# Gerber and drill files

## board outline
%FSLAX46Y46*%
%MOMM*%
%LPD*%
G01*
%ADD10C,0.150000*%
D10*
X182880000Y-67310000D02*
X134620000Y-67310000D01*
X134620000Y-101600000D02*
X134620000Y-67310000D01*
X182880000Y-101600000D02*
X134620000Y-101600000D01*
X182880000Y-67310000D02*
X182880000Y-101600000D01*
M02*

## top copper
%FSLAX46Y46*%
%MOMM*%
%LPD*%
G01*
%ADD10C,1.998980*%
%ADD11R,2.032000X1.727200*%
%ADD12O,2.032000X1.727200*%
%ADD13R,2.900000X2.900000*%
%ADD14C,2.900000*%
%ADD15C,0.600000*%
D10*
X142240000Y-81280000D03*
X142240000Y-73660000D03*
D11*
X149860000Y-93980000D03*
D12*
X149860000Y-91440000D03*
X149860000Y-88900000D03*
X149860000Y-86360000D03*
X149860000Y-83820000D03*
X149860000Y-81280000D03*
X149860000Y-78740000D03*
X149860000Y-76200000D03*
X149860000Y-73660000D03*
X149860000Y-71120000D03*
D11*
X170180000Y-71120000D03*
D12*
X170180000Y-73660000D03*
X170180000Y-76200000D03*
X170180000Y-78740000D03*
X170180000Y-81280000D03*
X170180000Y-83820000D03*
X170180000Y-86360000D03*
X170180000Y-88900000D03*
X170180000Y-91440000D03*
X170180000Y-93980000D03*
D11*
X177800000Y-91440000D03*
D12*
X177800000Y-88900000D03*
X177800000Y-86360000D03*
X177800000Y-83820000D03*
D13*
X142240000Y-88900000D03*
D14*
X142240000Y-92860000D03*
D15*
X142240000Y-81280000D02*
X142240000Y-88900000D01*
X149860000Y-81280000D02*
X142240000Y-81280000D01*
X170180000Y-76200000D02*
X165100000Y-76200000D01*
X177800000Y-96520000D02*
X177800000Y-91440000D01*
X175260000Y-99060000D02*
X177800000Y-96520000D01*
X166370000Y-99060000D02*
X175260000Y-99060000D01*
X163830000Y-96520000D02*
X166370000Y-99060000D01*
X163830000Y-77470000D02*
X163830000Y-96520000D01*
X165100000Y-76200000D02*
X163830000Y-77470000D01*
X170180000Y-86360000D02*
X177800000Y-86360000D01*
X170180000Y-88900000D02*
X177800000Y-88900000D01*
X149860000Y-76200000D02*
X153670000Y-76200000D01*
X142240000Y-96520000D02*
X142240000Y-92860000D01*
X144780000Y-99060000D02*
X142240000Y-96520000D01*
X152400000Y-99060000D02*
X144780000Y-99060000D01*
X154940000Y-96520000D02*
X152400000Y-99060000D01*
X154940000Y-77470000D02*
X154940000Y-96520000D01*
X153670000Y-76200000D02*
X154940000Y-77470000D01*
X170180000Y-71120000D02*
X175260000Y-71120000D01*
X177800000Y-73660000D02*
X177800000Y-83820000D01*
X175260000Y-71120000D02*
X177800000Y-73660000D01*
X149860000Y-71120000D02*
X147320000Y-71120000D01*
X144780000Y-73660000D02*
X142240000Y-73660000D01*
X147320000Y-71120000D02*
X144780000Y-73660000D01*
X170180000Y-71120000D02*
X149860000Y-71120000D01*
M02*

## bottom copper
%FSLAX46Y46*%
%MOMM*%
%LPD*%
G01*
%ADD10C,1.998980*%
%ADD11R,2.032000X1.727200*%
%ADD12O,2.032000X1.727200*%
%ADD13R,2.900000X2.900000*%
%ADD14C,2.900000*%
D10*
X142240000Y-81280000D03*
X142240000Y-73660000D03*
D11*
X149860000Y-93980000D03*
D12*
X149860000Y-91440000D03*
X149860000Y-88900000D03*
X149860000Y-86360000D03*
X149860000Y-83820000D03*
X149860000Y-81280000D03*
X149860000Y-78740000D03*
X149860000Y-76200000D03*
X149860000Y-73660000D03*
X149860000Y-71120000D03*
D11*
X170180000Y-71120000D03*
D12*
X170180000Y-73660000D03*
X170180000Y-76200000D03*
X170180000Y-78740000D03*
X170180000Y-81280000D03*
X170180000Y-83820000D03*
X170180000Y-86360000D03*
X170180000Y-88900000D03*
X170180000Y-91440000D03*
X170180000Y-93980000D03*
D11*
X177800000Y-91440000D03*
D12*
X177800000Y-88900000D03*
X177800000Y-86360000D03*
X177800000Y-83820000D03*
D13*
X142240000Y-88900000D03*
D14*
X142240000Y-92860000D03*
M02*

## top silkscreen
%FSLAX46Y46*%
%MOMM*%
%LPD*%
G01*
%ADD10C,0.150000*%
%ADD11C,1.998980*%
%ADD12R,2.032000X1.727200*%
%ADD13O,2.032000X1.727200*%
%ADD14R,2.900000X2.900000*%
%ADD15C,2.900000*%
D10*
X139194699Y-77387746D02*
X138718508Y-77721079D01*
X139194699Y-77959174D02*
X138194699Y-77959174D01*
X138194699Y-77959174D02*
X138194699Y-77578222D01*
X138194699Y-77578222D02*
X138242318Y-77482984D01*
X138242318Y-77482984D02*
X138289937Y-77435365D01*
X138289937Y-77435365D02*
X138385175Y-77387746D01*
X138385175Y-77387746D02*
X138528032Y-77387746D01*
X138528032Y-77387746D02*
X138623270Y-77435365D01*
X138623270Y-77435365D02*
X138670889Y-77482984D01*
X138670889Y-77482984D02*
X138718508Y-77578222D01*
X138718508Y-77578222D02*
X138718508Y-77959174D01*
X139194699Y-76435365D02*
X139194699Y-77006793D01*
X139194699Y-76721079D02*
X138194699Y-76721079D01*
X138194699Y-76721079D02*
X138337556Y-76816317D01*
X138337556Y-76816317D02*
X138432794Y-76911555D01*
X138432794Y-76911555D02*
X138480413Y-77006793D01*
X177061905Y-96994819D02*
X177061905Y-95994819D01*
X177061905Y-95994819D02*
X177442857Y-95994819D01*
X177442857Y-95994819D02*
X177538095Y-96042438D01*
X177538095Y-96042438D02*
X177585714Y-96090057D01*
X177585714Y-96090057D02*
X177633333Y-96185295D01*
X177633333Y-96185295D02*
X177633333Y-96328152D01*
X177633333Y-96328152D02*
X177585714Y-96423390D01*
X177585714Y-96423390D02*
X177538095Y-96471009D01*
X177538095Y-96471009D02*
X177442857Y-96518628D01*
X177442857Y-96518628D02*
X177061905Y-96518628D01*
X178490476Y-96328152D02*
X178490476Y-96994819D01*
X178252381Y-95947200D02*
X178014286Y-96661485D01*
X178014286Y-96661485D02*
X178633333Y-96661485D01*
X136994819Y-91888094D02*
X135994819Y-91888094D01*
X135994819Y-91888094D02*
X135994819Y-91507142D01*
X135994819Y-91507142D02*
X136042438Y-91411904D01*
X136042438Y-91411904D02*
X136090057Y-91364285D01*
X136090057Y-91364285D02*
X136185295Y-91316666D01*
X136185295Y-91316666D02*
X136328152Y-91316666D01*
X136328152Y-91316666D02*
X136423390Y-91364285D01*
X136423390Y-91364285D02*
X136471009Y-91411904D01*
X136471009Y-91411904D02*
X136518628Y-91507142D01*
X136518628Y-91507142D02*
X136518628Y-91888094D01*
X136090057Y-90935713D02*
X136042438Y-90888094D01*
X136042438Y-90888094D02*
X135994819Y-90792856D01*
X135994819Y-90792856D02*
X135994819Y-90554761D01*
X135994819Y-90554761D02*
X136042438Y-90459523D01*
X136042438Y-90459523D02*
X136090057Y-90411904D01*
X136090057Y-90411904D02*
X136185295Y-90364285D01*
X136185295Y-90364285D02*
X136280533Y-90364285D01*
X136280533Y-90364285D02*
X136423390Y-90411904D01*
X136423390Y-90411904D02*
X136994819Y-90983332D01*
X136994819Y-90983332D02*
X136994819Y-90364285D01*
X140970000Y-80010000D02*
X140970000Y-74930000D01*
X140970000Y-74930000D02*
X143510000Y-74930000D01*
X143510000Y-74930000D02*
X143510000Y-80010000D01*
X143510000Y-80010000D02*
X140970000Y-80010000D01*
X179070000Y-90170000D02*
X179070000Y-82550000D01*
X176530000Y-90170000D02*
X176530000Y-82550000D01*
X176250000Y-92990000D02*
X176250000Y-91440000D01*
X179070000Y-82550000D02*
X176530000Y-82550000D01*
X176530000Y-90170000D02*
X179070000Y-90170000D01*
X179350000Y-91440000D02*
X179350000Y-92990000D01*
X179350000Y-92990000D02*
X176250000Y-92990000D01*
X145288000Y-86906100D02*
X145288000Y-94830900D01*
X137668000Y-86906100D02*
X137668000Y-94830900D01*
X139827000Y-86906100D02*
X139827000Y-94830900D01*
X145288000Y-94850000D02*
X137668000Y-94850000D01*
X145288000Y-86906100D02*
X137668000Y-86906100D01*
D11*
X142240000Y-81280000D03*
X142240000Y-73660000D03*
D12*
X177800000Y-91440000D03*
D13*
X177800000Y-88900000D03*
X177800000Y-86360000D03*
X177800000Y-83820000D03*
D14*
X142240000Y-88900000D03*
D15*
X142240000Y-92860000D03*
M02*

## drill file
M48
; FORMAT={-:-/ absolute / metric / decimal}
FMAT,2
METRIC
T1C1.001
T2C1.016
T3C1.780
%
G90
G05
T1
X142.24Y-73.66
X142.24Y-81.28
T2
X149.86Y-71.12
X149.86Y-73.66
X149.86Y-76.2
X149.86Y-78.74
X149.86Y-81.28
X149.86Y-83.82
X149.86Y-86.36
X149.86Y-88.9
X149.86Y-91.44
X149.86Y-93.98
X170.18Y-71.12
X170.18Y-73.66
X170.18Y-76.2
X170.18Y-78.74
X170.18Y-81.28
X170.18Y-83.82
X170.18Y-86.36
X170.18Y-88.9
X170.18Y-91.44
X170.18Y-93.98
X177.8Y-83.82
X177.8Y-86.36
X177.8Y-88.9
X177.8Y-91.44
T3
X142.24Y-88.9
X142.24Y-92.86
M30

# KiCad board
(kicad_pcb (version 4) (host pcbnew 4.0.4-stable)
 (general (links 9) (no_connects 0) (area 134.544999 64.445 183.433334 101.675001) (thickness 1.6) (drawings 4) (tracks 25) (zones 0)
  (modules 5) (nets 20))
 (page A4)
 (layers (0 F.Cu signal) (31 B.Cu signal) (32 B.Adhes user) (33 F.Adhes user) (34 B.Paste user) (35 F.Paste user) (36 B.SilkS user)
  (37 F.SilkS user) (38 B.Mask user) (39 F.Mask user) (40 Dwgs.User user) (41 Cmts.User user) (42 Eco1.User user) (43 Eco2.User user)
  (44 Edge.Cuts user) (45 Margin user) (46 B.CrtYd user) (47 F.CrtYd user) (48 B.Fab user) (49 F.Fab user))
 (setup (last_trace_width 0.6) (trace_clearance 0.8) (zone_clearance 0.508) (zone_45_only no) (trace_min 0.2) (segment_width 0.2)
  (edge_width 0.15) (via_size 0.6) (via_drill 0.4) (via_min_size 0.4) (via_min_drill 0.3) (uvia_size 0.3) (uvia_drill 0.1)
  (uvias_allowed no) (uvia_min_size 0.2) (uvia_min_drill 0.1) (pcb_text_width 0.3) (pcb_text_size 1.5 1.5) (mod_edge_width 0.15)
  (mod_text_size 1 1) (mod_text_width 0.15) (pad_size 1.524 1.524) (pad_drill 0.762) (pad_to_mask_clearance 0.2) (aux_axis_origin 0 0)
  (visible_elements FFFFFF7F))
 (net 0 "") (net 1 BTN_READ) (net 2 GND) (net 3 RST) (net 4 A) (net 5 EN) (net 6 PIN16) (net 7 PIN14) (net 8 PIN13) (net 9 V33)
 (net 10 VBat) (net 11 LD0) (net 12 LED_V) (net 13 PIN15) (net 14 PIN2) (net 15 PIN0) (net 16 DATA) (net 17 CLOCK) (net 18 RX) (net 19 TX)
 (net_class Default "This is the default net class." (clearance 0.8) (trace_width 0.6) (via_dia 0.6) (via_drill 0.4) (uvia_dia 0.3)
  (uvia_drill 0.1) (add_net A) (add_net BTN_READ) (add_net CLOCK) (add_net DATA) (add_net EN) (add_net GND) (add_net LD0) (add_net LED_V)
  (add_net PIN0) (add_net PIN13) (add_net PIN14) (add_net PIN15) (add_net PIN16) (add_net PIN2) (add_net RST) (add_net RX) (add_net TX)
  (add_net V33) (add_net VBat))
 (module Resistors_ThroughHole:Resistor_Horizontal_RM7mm (layer F.Cu) (at 142.24 81.28 90)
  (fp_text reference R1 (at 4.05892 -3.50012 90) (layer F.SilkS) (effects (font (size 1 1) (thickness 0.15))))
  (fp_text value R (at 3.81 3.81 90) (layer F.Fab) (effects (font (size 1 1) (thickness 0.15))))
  (fp_line (start 1.27 -1.27) (end 6.35 -1.27) (layer F.SilkS) (width 0.15))
  (fp_line (start 6.35 -1.27) (end 6.35 1.27) (layer F.SilkS) (width 0.15))
  (fp_line (start 6.35 1.27) (end 1.27 1.27) (layer F.SilkS) (width 0.15))
  (fp_line (start 1.27 1.27) (end 1.27 -1.27) (layer F.SilkS) (width 0.15))
  (pad 1 thru_hole circle (at 0 0 90) (size 1.99898 1.99898) (drill 1.00076) (layers *.Cu *.SilkS *.Mask) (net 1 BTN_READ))
  (pad 2 thru_hole circle (at 7.62 0 90) (size 1.99898 1.99898) (drill 1.00076) (layers *.Cu *.SilkS *.Mask) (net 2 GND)))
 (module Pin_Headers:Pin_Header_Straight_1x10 (layer B.Cu) (at 149.86 93.98)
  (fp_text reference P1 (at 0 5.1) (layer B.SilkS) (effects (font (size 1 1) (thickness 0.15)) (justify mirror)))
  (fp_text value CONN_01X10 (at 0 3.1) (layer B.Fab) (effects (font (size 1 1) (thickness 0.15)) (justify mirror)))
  (pad 1 thru_hole rect (at 0 0) (size 2.032 1.7272) (drill 1.016) (layers *.Cu *.Mask B.SilkS) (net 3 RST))
  (pad 2 thru_hole oval (at 0 -2.54) (size 2.032 1.7272) (drill 1.016) (layers *.Cu *.Mask B.SilkS) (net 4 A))
  (pad 3 thru_hole oval (at 0 -5.08) (size 2.032 1.7272) (drill 1.016) (layers *.Cu *.Mask B.SilkS) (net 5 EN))
  (pad 4 thru_hole oval (at 0 -7.62) (size 2.032 1.7272) (drill 1.016) (layers *.Cu *.Mask B.SilkS) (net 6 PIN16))
  (pad 5 thru_hole oval (at 0 -10.16) (size 2.032 1.7272) (drill 1.016) (layers *.Cu *.Mask B.SilkS) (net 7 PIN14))
  (pad 6 thru_hole oval (at 0 -12.7) (size 2.032 1.7272) (drill 1.016) (layers *.Cu *.Mask B.SilkS) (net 1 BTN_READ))
  (pad 7 thru_hole oval (at 0 -15.24) (size 2.032 1.7272) (drill 1.016) (layers *.Cu *.Mask B.SilkS) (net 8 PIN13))
  (pad 8 thru_hole oval (at 0 -17.78) (size 2.032 1.7272) (drill 1.016) (layers *.Cu *.Mask B.SilkS) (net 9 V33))
  (pad 9 thru_hole oval (at 0 -20.32) (size 2.032 1.7272) (drill 1.016) (layers *.Cu *.Mask B.SilkS) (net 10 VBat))
  (pad 10 thru_hole oval (at 0 -22.86) (size 2.032 1.7272) (drill 1.016) (layers *.Cu *.Mask B.SilkS) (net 2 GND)))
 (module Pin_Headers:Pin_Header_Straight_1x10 (layer B.Cu) (at 170.18 71.12 180)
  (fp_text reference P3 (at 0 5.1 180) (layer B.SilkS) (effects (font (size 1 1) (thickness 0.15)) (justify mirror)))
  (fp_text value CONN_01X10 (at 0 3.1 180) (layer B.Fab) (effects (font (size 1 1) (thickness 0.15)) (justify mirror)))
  (pad 1 thru_hole rect (at 0 0 180) (size 2.032 1.7272) (drill 1.016) (layers *.Cu *.Mask B.SilkS) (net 2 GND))
  (pad 2 thru_hole oval (at 0 -2.54 180) (size 2.032 1.7272) (drill 1.016) (layers *.Cu *.Mask B.SilkS) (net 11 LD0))
  (pad 3 thru_hole oval (at 0 -5.08 180) (size 2.032 1.7272) (drill 1.016) (layers *.Cu *.Mask B.SilkS) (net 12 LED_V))
  (pad 4 thru_hole oval (at 0 -7.62 180) (size 2.032 1.7272) (drill 1.016) (layers *.Cu *.Mask B.SilkS) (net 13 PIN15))
  (pad 5 thru_hole oval (at 0 -10.16 180) (size 2.032 1.7272) (drill 1.016) (layers *.Cu *.Mask B.SilkS) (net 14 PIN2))
  (pad 6 thru_hole oval (at 0 -12.7 180) (size 2.032 1.7272) (drill 1.016) (layers *.Cu *.Mask B.SilkS) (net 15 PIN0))
  (pad 7 thru_hole oval (at 0 -15.24 180) (size 2.032 1.7272) (drill 1.016) (layers *.Cu *.Mask B.SilkS) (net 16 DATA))
  (pad 8 thru_hole oval (at 0 -17.78 180) (size 2.032 1.7272) (drill 1.016) (layers *.Cu *.Mask B.SilkS) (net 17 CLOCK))
  (pad 9 thru_hole oval (at 0 -20.32 180) (size 2.032 1.7272) (drill 1.016) (layers *.Cu *.Mask B.SilkS) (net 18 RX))
  (pad 10 thru_hole oval (at 0 -22.86 180) (size 2.032 1.7272) (drill 1.016) (layers *.Cu *.Mask B.SilkS) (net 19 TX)))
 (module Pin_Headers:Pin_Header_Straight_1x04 (layer F.Cu) (at 177.8 91.44 180)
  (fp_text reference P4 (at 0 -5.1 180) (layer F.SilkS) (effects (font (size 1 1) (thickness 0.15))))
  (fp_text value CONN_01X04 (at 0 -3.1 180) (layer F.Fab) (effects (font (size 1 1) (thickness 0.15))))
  (fp_line (start -1.27 1.27) (end -1.27 8.89) (layer F.SilkS) (width 0.15))
  (fp_line (start 1.27 1.27) (end 1.27 8.89) (layer F.SilkS) (width 0.15))
  (fp_line (start 1.55 -1.55) (end 1.55 0) (layer F.SilkS) (width 0.15))
  (fp_line (start -1.27 8.89) (end 1.27 8.89) (layer F.SilkS) (width 0.15))
  (fp_line (start 1.27 1.27) (end -1.27 1.27) (layer F.SilkS) (width 0.15))
  (fp_line (start -1.55 0) (end -1.55 -1.55) (layer F.SilkS) (width 0.15))
  (fp_line (start -1.55 -1.55) (end 1.55 -1.55) (layer F.SilkS) (width 0.15))
  (pad 1 thru_hole rect (at 0 0 180) (size 2.032 1.7272) (drill 1.016) (layers *.Cu *.Mask F.SilkS) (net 12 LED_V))
  (pad 2 thru_hole oval (at 0 2.54 180) (size 2.032 1.7272) (drill 1.016) (layers *.Cu *.Mask F.SilkS) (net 17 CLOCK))
  (pad 3 thru_hole oval (at 0 5.08 180) (size 2.032 1.7272) (drill 1.016) (layers *.Cu *.Mask F.SilkS) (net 16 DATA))
  (pad 4 thru_hole oval (at 0 7.62 180) (size 2.032 1.7272) (drill 1.016) (layers *.Cu *.Mask F.SilkS) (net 2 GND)))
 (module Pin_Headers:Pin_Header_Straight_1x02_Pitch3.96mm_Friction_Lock (layer F.Cu) (at 142.24 88.9 270)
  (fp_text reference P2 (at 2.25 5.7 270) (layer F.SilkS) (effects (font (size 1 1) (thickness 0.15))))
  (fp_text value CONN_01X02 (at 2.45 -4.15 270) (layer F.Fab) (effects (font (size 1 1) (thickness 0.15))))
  (fp_line (start -1.9939 -3.048) (end 5.9309 -3.048) (layer F.SilkS) (width 0.15))
  (fp_line (start -1.9939 4.572) (end 5.9309 4.572) (layer F.SilkS) (width 0.15))
  (fp_line (start -1.9939 2.413) (end 5.9309 2.413) (layer F.SilkS) (width 0.15))
  (fp_line (start 5.95 -3.048) (end 5.95 4.572) (layer F.SilkS) (width 0.15))
  (fp_line (start -1.9939 -3.048) (end -1.9939 4.572) (layer F.SilkS) (width 0.15))
  (pad 1 thru_hole rect (at 0 0 270) (size 2.9 2.9) (drill 1.78) (layers *.Cu *.Mask F.SilkS) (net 1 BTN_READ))
  (pad 2 thru_hole circle (at 3.96 0 270) (size 2.9 2.9) (drill 1.78) (layers *.Cu *.Mask F.SilkS) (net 9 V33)))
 (gr_line (start 182.88 67.31) (end 134.62 67.31) (angle 90) (layer Edge.Cuts) (width 0.15))
 (gr_line (start 134.62 101.6) (end 134.62 67.31) (angle 90) (layer Edge.Cuts) (width 0.15))
 (gr_line (start 182.88 101.6) (end 134.62 101.6) (angle 90) (layer Edge.Cuts) (width 0.15))
 (gr_line (start 182.88 67.31) (end 182.88 101.6) (angle 90) (layer Edge.Cuts) (width 0.15))
 (segment (start 142.24 81.28) (end 142.24 88.9) (width 0.6) (layer F.Cu) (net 1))
 (segment (start 149.86 81.28) (end 142.24 81.28) (width 0.6) (layer F.Cu) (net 1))
 (segment (start 170.18 76.2) (end 165.1 76.2) (width 0.6) (layer F.Cu) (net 12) (status 400000))
 (segment (start 177.8 96.52) (end 177.8 91.44) (width 0.6) (layer F.Cu) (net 12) (status 800000))
 (segment (start 175.26 99.06) (end 177.8 96.52) (width 0.6) (layer F.Cu) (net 12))
 (segment (start 166.37 99.06) (end 175.26 99.06) (width 0.6) (layer F.Cu) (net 12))
 (segment (start 163.83 96.52) (end 166.37 99.06) (width 0.6) (layer F.Cu) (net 12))
 (segment (start 163.83 77.47) (end 163.83 96.52) (width 0.6) (layer F.Cu) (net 12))
 (segment (start 165.1 76.2) (end 163.83 77.47) (width 0.6) (layer F.Cu) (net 12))
 (segment (start 170.18 86.36) (end 177.8 86.36) (width 0.6) (layer F.Cu) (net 16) (status C00000))
 (segment (start 170.18 88.9) (end 177.8 88.9) (width 0.6) (layer F.Cu) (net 17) (status C00000))
 (segment (start 149.86 76.2) (end 153.67 76.2) (width 0.6) (layer F.Cu) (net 9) (status 400000))
 (segment (start 142.24 96.52) (end 142.24 92.86) (width 0.6) (layer F.Cu) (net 9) (status 800000))
 (segment (start 144.78 99.06) (end 142.24 96.52) (width 0.6) (layer F.Cu) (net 9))
 (segment (start 152.4 99.06) (end 144.78 99.06) (width 0.6) (layer F.Cu) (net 9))
 (segment (start 154.94 96.52) (end 152.4 99.06) (width 0.6) (layer F.Cu) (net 9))
 (segment (start 154.94 77.47) (end 154.94 96.52) (width 0.6) (layer F.Cu) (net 9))
 (segment (start 153.67 76.2) (end 154.94 77.47) (width 0.6) (layer F.Cu) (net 9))
 (segment (start 170.18 71.12) (end 175.26 71.12) (width 0.6) (layer F.Cu) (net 2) (status 400000))
 (segment (start 177.8 73.66) (end 177.8 83.82) (width 0.6) (layer F.Cu) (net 2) (status 800000))
 (segment (start 175.26 71.12) (end 177.8 73.66) (width 0.6) (layer F.Cu) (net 2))
 (segment (start 149.86 71.12) (end 147.32 71.12) (width 0.6) (layer F.Cu) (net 2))
 (segment (start 144.78 73.66) (end 142.24 73.66) (width 0.6) (layer F.Cu) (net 2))
 (segment (start 147.32 71.12) (end 144.78 73.66) (width 0.6) (layer F.Cu) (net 2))
 (segment (start 170.18 71.12) (end 149.86 71.12) (width 0.6) (layer F.Cu) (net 2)))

